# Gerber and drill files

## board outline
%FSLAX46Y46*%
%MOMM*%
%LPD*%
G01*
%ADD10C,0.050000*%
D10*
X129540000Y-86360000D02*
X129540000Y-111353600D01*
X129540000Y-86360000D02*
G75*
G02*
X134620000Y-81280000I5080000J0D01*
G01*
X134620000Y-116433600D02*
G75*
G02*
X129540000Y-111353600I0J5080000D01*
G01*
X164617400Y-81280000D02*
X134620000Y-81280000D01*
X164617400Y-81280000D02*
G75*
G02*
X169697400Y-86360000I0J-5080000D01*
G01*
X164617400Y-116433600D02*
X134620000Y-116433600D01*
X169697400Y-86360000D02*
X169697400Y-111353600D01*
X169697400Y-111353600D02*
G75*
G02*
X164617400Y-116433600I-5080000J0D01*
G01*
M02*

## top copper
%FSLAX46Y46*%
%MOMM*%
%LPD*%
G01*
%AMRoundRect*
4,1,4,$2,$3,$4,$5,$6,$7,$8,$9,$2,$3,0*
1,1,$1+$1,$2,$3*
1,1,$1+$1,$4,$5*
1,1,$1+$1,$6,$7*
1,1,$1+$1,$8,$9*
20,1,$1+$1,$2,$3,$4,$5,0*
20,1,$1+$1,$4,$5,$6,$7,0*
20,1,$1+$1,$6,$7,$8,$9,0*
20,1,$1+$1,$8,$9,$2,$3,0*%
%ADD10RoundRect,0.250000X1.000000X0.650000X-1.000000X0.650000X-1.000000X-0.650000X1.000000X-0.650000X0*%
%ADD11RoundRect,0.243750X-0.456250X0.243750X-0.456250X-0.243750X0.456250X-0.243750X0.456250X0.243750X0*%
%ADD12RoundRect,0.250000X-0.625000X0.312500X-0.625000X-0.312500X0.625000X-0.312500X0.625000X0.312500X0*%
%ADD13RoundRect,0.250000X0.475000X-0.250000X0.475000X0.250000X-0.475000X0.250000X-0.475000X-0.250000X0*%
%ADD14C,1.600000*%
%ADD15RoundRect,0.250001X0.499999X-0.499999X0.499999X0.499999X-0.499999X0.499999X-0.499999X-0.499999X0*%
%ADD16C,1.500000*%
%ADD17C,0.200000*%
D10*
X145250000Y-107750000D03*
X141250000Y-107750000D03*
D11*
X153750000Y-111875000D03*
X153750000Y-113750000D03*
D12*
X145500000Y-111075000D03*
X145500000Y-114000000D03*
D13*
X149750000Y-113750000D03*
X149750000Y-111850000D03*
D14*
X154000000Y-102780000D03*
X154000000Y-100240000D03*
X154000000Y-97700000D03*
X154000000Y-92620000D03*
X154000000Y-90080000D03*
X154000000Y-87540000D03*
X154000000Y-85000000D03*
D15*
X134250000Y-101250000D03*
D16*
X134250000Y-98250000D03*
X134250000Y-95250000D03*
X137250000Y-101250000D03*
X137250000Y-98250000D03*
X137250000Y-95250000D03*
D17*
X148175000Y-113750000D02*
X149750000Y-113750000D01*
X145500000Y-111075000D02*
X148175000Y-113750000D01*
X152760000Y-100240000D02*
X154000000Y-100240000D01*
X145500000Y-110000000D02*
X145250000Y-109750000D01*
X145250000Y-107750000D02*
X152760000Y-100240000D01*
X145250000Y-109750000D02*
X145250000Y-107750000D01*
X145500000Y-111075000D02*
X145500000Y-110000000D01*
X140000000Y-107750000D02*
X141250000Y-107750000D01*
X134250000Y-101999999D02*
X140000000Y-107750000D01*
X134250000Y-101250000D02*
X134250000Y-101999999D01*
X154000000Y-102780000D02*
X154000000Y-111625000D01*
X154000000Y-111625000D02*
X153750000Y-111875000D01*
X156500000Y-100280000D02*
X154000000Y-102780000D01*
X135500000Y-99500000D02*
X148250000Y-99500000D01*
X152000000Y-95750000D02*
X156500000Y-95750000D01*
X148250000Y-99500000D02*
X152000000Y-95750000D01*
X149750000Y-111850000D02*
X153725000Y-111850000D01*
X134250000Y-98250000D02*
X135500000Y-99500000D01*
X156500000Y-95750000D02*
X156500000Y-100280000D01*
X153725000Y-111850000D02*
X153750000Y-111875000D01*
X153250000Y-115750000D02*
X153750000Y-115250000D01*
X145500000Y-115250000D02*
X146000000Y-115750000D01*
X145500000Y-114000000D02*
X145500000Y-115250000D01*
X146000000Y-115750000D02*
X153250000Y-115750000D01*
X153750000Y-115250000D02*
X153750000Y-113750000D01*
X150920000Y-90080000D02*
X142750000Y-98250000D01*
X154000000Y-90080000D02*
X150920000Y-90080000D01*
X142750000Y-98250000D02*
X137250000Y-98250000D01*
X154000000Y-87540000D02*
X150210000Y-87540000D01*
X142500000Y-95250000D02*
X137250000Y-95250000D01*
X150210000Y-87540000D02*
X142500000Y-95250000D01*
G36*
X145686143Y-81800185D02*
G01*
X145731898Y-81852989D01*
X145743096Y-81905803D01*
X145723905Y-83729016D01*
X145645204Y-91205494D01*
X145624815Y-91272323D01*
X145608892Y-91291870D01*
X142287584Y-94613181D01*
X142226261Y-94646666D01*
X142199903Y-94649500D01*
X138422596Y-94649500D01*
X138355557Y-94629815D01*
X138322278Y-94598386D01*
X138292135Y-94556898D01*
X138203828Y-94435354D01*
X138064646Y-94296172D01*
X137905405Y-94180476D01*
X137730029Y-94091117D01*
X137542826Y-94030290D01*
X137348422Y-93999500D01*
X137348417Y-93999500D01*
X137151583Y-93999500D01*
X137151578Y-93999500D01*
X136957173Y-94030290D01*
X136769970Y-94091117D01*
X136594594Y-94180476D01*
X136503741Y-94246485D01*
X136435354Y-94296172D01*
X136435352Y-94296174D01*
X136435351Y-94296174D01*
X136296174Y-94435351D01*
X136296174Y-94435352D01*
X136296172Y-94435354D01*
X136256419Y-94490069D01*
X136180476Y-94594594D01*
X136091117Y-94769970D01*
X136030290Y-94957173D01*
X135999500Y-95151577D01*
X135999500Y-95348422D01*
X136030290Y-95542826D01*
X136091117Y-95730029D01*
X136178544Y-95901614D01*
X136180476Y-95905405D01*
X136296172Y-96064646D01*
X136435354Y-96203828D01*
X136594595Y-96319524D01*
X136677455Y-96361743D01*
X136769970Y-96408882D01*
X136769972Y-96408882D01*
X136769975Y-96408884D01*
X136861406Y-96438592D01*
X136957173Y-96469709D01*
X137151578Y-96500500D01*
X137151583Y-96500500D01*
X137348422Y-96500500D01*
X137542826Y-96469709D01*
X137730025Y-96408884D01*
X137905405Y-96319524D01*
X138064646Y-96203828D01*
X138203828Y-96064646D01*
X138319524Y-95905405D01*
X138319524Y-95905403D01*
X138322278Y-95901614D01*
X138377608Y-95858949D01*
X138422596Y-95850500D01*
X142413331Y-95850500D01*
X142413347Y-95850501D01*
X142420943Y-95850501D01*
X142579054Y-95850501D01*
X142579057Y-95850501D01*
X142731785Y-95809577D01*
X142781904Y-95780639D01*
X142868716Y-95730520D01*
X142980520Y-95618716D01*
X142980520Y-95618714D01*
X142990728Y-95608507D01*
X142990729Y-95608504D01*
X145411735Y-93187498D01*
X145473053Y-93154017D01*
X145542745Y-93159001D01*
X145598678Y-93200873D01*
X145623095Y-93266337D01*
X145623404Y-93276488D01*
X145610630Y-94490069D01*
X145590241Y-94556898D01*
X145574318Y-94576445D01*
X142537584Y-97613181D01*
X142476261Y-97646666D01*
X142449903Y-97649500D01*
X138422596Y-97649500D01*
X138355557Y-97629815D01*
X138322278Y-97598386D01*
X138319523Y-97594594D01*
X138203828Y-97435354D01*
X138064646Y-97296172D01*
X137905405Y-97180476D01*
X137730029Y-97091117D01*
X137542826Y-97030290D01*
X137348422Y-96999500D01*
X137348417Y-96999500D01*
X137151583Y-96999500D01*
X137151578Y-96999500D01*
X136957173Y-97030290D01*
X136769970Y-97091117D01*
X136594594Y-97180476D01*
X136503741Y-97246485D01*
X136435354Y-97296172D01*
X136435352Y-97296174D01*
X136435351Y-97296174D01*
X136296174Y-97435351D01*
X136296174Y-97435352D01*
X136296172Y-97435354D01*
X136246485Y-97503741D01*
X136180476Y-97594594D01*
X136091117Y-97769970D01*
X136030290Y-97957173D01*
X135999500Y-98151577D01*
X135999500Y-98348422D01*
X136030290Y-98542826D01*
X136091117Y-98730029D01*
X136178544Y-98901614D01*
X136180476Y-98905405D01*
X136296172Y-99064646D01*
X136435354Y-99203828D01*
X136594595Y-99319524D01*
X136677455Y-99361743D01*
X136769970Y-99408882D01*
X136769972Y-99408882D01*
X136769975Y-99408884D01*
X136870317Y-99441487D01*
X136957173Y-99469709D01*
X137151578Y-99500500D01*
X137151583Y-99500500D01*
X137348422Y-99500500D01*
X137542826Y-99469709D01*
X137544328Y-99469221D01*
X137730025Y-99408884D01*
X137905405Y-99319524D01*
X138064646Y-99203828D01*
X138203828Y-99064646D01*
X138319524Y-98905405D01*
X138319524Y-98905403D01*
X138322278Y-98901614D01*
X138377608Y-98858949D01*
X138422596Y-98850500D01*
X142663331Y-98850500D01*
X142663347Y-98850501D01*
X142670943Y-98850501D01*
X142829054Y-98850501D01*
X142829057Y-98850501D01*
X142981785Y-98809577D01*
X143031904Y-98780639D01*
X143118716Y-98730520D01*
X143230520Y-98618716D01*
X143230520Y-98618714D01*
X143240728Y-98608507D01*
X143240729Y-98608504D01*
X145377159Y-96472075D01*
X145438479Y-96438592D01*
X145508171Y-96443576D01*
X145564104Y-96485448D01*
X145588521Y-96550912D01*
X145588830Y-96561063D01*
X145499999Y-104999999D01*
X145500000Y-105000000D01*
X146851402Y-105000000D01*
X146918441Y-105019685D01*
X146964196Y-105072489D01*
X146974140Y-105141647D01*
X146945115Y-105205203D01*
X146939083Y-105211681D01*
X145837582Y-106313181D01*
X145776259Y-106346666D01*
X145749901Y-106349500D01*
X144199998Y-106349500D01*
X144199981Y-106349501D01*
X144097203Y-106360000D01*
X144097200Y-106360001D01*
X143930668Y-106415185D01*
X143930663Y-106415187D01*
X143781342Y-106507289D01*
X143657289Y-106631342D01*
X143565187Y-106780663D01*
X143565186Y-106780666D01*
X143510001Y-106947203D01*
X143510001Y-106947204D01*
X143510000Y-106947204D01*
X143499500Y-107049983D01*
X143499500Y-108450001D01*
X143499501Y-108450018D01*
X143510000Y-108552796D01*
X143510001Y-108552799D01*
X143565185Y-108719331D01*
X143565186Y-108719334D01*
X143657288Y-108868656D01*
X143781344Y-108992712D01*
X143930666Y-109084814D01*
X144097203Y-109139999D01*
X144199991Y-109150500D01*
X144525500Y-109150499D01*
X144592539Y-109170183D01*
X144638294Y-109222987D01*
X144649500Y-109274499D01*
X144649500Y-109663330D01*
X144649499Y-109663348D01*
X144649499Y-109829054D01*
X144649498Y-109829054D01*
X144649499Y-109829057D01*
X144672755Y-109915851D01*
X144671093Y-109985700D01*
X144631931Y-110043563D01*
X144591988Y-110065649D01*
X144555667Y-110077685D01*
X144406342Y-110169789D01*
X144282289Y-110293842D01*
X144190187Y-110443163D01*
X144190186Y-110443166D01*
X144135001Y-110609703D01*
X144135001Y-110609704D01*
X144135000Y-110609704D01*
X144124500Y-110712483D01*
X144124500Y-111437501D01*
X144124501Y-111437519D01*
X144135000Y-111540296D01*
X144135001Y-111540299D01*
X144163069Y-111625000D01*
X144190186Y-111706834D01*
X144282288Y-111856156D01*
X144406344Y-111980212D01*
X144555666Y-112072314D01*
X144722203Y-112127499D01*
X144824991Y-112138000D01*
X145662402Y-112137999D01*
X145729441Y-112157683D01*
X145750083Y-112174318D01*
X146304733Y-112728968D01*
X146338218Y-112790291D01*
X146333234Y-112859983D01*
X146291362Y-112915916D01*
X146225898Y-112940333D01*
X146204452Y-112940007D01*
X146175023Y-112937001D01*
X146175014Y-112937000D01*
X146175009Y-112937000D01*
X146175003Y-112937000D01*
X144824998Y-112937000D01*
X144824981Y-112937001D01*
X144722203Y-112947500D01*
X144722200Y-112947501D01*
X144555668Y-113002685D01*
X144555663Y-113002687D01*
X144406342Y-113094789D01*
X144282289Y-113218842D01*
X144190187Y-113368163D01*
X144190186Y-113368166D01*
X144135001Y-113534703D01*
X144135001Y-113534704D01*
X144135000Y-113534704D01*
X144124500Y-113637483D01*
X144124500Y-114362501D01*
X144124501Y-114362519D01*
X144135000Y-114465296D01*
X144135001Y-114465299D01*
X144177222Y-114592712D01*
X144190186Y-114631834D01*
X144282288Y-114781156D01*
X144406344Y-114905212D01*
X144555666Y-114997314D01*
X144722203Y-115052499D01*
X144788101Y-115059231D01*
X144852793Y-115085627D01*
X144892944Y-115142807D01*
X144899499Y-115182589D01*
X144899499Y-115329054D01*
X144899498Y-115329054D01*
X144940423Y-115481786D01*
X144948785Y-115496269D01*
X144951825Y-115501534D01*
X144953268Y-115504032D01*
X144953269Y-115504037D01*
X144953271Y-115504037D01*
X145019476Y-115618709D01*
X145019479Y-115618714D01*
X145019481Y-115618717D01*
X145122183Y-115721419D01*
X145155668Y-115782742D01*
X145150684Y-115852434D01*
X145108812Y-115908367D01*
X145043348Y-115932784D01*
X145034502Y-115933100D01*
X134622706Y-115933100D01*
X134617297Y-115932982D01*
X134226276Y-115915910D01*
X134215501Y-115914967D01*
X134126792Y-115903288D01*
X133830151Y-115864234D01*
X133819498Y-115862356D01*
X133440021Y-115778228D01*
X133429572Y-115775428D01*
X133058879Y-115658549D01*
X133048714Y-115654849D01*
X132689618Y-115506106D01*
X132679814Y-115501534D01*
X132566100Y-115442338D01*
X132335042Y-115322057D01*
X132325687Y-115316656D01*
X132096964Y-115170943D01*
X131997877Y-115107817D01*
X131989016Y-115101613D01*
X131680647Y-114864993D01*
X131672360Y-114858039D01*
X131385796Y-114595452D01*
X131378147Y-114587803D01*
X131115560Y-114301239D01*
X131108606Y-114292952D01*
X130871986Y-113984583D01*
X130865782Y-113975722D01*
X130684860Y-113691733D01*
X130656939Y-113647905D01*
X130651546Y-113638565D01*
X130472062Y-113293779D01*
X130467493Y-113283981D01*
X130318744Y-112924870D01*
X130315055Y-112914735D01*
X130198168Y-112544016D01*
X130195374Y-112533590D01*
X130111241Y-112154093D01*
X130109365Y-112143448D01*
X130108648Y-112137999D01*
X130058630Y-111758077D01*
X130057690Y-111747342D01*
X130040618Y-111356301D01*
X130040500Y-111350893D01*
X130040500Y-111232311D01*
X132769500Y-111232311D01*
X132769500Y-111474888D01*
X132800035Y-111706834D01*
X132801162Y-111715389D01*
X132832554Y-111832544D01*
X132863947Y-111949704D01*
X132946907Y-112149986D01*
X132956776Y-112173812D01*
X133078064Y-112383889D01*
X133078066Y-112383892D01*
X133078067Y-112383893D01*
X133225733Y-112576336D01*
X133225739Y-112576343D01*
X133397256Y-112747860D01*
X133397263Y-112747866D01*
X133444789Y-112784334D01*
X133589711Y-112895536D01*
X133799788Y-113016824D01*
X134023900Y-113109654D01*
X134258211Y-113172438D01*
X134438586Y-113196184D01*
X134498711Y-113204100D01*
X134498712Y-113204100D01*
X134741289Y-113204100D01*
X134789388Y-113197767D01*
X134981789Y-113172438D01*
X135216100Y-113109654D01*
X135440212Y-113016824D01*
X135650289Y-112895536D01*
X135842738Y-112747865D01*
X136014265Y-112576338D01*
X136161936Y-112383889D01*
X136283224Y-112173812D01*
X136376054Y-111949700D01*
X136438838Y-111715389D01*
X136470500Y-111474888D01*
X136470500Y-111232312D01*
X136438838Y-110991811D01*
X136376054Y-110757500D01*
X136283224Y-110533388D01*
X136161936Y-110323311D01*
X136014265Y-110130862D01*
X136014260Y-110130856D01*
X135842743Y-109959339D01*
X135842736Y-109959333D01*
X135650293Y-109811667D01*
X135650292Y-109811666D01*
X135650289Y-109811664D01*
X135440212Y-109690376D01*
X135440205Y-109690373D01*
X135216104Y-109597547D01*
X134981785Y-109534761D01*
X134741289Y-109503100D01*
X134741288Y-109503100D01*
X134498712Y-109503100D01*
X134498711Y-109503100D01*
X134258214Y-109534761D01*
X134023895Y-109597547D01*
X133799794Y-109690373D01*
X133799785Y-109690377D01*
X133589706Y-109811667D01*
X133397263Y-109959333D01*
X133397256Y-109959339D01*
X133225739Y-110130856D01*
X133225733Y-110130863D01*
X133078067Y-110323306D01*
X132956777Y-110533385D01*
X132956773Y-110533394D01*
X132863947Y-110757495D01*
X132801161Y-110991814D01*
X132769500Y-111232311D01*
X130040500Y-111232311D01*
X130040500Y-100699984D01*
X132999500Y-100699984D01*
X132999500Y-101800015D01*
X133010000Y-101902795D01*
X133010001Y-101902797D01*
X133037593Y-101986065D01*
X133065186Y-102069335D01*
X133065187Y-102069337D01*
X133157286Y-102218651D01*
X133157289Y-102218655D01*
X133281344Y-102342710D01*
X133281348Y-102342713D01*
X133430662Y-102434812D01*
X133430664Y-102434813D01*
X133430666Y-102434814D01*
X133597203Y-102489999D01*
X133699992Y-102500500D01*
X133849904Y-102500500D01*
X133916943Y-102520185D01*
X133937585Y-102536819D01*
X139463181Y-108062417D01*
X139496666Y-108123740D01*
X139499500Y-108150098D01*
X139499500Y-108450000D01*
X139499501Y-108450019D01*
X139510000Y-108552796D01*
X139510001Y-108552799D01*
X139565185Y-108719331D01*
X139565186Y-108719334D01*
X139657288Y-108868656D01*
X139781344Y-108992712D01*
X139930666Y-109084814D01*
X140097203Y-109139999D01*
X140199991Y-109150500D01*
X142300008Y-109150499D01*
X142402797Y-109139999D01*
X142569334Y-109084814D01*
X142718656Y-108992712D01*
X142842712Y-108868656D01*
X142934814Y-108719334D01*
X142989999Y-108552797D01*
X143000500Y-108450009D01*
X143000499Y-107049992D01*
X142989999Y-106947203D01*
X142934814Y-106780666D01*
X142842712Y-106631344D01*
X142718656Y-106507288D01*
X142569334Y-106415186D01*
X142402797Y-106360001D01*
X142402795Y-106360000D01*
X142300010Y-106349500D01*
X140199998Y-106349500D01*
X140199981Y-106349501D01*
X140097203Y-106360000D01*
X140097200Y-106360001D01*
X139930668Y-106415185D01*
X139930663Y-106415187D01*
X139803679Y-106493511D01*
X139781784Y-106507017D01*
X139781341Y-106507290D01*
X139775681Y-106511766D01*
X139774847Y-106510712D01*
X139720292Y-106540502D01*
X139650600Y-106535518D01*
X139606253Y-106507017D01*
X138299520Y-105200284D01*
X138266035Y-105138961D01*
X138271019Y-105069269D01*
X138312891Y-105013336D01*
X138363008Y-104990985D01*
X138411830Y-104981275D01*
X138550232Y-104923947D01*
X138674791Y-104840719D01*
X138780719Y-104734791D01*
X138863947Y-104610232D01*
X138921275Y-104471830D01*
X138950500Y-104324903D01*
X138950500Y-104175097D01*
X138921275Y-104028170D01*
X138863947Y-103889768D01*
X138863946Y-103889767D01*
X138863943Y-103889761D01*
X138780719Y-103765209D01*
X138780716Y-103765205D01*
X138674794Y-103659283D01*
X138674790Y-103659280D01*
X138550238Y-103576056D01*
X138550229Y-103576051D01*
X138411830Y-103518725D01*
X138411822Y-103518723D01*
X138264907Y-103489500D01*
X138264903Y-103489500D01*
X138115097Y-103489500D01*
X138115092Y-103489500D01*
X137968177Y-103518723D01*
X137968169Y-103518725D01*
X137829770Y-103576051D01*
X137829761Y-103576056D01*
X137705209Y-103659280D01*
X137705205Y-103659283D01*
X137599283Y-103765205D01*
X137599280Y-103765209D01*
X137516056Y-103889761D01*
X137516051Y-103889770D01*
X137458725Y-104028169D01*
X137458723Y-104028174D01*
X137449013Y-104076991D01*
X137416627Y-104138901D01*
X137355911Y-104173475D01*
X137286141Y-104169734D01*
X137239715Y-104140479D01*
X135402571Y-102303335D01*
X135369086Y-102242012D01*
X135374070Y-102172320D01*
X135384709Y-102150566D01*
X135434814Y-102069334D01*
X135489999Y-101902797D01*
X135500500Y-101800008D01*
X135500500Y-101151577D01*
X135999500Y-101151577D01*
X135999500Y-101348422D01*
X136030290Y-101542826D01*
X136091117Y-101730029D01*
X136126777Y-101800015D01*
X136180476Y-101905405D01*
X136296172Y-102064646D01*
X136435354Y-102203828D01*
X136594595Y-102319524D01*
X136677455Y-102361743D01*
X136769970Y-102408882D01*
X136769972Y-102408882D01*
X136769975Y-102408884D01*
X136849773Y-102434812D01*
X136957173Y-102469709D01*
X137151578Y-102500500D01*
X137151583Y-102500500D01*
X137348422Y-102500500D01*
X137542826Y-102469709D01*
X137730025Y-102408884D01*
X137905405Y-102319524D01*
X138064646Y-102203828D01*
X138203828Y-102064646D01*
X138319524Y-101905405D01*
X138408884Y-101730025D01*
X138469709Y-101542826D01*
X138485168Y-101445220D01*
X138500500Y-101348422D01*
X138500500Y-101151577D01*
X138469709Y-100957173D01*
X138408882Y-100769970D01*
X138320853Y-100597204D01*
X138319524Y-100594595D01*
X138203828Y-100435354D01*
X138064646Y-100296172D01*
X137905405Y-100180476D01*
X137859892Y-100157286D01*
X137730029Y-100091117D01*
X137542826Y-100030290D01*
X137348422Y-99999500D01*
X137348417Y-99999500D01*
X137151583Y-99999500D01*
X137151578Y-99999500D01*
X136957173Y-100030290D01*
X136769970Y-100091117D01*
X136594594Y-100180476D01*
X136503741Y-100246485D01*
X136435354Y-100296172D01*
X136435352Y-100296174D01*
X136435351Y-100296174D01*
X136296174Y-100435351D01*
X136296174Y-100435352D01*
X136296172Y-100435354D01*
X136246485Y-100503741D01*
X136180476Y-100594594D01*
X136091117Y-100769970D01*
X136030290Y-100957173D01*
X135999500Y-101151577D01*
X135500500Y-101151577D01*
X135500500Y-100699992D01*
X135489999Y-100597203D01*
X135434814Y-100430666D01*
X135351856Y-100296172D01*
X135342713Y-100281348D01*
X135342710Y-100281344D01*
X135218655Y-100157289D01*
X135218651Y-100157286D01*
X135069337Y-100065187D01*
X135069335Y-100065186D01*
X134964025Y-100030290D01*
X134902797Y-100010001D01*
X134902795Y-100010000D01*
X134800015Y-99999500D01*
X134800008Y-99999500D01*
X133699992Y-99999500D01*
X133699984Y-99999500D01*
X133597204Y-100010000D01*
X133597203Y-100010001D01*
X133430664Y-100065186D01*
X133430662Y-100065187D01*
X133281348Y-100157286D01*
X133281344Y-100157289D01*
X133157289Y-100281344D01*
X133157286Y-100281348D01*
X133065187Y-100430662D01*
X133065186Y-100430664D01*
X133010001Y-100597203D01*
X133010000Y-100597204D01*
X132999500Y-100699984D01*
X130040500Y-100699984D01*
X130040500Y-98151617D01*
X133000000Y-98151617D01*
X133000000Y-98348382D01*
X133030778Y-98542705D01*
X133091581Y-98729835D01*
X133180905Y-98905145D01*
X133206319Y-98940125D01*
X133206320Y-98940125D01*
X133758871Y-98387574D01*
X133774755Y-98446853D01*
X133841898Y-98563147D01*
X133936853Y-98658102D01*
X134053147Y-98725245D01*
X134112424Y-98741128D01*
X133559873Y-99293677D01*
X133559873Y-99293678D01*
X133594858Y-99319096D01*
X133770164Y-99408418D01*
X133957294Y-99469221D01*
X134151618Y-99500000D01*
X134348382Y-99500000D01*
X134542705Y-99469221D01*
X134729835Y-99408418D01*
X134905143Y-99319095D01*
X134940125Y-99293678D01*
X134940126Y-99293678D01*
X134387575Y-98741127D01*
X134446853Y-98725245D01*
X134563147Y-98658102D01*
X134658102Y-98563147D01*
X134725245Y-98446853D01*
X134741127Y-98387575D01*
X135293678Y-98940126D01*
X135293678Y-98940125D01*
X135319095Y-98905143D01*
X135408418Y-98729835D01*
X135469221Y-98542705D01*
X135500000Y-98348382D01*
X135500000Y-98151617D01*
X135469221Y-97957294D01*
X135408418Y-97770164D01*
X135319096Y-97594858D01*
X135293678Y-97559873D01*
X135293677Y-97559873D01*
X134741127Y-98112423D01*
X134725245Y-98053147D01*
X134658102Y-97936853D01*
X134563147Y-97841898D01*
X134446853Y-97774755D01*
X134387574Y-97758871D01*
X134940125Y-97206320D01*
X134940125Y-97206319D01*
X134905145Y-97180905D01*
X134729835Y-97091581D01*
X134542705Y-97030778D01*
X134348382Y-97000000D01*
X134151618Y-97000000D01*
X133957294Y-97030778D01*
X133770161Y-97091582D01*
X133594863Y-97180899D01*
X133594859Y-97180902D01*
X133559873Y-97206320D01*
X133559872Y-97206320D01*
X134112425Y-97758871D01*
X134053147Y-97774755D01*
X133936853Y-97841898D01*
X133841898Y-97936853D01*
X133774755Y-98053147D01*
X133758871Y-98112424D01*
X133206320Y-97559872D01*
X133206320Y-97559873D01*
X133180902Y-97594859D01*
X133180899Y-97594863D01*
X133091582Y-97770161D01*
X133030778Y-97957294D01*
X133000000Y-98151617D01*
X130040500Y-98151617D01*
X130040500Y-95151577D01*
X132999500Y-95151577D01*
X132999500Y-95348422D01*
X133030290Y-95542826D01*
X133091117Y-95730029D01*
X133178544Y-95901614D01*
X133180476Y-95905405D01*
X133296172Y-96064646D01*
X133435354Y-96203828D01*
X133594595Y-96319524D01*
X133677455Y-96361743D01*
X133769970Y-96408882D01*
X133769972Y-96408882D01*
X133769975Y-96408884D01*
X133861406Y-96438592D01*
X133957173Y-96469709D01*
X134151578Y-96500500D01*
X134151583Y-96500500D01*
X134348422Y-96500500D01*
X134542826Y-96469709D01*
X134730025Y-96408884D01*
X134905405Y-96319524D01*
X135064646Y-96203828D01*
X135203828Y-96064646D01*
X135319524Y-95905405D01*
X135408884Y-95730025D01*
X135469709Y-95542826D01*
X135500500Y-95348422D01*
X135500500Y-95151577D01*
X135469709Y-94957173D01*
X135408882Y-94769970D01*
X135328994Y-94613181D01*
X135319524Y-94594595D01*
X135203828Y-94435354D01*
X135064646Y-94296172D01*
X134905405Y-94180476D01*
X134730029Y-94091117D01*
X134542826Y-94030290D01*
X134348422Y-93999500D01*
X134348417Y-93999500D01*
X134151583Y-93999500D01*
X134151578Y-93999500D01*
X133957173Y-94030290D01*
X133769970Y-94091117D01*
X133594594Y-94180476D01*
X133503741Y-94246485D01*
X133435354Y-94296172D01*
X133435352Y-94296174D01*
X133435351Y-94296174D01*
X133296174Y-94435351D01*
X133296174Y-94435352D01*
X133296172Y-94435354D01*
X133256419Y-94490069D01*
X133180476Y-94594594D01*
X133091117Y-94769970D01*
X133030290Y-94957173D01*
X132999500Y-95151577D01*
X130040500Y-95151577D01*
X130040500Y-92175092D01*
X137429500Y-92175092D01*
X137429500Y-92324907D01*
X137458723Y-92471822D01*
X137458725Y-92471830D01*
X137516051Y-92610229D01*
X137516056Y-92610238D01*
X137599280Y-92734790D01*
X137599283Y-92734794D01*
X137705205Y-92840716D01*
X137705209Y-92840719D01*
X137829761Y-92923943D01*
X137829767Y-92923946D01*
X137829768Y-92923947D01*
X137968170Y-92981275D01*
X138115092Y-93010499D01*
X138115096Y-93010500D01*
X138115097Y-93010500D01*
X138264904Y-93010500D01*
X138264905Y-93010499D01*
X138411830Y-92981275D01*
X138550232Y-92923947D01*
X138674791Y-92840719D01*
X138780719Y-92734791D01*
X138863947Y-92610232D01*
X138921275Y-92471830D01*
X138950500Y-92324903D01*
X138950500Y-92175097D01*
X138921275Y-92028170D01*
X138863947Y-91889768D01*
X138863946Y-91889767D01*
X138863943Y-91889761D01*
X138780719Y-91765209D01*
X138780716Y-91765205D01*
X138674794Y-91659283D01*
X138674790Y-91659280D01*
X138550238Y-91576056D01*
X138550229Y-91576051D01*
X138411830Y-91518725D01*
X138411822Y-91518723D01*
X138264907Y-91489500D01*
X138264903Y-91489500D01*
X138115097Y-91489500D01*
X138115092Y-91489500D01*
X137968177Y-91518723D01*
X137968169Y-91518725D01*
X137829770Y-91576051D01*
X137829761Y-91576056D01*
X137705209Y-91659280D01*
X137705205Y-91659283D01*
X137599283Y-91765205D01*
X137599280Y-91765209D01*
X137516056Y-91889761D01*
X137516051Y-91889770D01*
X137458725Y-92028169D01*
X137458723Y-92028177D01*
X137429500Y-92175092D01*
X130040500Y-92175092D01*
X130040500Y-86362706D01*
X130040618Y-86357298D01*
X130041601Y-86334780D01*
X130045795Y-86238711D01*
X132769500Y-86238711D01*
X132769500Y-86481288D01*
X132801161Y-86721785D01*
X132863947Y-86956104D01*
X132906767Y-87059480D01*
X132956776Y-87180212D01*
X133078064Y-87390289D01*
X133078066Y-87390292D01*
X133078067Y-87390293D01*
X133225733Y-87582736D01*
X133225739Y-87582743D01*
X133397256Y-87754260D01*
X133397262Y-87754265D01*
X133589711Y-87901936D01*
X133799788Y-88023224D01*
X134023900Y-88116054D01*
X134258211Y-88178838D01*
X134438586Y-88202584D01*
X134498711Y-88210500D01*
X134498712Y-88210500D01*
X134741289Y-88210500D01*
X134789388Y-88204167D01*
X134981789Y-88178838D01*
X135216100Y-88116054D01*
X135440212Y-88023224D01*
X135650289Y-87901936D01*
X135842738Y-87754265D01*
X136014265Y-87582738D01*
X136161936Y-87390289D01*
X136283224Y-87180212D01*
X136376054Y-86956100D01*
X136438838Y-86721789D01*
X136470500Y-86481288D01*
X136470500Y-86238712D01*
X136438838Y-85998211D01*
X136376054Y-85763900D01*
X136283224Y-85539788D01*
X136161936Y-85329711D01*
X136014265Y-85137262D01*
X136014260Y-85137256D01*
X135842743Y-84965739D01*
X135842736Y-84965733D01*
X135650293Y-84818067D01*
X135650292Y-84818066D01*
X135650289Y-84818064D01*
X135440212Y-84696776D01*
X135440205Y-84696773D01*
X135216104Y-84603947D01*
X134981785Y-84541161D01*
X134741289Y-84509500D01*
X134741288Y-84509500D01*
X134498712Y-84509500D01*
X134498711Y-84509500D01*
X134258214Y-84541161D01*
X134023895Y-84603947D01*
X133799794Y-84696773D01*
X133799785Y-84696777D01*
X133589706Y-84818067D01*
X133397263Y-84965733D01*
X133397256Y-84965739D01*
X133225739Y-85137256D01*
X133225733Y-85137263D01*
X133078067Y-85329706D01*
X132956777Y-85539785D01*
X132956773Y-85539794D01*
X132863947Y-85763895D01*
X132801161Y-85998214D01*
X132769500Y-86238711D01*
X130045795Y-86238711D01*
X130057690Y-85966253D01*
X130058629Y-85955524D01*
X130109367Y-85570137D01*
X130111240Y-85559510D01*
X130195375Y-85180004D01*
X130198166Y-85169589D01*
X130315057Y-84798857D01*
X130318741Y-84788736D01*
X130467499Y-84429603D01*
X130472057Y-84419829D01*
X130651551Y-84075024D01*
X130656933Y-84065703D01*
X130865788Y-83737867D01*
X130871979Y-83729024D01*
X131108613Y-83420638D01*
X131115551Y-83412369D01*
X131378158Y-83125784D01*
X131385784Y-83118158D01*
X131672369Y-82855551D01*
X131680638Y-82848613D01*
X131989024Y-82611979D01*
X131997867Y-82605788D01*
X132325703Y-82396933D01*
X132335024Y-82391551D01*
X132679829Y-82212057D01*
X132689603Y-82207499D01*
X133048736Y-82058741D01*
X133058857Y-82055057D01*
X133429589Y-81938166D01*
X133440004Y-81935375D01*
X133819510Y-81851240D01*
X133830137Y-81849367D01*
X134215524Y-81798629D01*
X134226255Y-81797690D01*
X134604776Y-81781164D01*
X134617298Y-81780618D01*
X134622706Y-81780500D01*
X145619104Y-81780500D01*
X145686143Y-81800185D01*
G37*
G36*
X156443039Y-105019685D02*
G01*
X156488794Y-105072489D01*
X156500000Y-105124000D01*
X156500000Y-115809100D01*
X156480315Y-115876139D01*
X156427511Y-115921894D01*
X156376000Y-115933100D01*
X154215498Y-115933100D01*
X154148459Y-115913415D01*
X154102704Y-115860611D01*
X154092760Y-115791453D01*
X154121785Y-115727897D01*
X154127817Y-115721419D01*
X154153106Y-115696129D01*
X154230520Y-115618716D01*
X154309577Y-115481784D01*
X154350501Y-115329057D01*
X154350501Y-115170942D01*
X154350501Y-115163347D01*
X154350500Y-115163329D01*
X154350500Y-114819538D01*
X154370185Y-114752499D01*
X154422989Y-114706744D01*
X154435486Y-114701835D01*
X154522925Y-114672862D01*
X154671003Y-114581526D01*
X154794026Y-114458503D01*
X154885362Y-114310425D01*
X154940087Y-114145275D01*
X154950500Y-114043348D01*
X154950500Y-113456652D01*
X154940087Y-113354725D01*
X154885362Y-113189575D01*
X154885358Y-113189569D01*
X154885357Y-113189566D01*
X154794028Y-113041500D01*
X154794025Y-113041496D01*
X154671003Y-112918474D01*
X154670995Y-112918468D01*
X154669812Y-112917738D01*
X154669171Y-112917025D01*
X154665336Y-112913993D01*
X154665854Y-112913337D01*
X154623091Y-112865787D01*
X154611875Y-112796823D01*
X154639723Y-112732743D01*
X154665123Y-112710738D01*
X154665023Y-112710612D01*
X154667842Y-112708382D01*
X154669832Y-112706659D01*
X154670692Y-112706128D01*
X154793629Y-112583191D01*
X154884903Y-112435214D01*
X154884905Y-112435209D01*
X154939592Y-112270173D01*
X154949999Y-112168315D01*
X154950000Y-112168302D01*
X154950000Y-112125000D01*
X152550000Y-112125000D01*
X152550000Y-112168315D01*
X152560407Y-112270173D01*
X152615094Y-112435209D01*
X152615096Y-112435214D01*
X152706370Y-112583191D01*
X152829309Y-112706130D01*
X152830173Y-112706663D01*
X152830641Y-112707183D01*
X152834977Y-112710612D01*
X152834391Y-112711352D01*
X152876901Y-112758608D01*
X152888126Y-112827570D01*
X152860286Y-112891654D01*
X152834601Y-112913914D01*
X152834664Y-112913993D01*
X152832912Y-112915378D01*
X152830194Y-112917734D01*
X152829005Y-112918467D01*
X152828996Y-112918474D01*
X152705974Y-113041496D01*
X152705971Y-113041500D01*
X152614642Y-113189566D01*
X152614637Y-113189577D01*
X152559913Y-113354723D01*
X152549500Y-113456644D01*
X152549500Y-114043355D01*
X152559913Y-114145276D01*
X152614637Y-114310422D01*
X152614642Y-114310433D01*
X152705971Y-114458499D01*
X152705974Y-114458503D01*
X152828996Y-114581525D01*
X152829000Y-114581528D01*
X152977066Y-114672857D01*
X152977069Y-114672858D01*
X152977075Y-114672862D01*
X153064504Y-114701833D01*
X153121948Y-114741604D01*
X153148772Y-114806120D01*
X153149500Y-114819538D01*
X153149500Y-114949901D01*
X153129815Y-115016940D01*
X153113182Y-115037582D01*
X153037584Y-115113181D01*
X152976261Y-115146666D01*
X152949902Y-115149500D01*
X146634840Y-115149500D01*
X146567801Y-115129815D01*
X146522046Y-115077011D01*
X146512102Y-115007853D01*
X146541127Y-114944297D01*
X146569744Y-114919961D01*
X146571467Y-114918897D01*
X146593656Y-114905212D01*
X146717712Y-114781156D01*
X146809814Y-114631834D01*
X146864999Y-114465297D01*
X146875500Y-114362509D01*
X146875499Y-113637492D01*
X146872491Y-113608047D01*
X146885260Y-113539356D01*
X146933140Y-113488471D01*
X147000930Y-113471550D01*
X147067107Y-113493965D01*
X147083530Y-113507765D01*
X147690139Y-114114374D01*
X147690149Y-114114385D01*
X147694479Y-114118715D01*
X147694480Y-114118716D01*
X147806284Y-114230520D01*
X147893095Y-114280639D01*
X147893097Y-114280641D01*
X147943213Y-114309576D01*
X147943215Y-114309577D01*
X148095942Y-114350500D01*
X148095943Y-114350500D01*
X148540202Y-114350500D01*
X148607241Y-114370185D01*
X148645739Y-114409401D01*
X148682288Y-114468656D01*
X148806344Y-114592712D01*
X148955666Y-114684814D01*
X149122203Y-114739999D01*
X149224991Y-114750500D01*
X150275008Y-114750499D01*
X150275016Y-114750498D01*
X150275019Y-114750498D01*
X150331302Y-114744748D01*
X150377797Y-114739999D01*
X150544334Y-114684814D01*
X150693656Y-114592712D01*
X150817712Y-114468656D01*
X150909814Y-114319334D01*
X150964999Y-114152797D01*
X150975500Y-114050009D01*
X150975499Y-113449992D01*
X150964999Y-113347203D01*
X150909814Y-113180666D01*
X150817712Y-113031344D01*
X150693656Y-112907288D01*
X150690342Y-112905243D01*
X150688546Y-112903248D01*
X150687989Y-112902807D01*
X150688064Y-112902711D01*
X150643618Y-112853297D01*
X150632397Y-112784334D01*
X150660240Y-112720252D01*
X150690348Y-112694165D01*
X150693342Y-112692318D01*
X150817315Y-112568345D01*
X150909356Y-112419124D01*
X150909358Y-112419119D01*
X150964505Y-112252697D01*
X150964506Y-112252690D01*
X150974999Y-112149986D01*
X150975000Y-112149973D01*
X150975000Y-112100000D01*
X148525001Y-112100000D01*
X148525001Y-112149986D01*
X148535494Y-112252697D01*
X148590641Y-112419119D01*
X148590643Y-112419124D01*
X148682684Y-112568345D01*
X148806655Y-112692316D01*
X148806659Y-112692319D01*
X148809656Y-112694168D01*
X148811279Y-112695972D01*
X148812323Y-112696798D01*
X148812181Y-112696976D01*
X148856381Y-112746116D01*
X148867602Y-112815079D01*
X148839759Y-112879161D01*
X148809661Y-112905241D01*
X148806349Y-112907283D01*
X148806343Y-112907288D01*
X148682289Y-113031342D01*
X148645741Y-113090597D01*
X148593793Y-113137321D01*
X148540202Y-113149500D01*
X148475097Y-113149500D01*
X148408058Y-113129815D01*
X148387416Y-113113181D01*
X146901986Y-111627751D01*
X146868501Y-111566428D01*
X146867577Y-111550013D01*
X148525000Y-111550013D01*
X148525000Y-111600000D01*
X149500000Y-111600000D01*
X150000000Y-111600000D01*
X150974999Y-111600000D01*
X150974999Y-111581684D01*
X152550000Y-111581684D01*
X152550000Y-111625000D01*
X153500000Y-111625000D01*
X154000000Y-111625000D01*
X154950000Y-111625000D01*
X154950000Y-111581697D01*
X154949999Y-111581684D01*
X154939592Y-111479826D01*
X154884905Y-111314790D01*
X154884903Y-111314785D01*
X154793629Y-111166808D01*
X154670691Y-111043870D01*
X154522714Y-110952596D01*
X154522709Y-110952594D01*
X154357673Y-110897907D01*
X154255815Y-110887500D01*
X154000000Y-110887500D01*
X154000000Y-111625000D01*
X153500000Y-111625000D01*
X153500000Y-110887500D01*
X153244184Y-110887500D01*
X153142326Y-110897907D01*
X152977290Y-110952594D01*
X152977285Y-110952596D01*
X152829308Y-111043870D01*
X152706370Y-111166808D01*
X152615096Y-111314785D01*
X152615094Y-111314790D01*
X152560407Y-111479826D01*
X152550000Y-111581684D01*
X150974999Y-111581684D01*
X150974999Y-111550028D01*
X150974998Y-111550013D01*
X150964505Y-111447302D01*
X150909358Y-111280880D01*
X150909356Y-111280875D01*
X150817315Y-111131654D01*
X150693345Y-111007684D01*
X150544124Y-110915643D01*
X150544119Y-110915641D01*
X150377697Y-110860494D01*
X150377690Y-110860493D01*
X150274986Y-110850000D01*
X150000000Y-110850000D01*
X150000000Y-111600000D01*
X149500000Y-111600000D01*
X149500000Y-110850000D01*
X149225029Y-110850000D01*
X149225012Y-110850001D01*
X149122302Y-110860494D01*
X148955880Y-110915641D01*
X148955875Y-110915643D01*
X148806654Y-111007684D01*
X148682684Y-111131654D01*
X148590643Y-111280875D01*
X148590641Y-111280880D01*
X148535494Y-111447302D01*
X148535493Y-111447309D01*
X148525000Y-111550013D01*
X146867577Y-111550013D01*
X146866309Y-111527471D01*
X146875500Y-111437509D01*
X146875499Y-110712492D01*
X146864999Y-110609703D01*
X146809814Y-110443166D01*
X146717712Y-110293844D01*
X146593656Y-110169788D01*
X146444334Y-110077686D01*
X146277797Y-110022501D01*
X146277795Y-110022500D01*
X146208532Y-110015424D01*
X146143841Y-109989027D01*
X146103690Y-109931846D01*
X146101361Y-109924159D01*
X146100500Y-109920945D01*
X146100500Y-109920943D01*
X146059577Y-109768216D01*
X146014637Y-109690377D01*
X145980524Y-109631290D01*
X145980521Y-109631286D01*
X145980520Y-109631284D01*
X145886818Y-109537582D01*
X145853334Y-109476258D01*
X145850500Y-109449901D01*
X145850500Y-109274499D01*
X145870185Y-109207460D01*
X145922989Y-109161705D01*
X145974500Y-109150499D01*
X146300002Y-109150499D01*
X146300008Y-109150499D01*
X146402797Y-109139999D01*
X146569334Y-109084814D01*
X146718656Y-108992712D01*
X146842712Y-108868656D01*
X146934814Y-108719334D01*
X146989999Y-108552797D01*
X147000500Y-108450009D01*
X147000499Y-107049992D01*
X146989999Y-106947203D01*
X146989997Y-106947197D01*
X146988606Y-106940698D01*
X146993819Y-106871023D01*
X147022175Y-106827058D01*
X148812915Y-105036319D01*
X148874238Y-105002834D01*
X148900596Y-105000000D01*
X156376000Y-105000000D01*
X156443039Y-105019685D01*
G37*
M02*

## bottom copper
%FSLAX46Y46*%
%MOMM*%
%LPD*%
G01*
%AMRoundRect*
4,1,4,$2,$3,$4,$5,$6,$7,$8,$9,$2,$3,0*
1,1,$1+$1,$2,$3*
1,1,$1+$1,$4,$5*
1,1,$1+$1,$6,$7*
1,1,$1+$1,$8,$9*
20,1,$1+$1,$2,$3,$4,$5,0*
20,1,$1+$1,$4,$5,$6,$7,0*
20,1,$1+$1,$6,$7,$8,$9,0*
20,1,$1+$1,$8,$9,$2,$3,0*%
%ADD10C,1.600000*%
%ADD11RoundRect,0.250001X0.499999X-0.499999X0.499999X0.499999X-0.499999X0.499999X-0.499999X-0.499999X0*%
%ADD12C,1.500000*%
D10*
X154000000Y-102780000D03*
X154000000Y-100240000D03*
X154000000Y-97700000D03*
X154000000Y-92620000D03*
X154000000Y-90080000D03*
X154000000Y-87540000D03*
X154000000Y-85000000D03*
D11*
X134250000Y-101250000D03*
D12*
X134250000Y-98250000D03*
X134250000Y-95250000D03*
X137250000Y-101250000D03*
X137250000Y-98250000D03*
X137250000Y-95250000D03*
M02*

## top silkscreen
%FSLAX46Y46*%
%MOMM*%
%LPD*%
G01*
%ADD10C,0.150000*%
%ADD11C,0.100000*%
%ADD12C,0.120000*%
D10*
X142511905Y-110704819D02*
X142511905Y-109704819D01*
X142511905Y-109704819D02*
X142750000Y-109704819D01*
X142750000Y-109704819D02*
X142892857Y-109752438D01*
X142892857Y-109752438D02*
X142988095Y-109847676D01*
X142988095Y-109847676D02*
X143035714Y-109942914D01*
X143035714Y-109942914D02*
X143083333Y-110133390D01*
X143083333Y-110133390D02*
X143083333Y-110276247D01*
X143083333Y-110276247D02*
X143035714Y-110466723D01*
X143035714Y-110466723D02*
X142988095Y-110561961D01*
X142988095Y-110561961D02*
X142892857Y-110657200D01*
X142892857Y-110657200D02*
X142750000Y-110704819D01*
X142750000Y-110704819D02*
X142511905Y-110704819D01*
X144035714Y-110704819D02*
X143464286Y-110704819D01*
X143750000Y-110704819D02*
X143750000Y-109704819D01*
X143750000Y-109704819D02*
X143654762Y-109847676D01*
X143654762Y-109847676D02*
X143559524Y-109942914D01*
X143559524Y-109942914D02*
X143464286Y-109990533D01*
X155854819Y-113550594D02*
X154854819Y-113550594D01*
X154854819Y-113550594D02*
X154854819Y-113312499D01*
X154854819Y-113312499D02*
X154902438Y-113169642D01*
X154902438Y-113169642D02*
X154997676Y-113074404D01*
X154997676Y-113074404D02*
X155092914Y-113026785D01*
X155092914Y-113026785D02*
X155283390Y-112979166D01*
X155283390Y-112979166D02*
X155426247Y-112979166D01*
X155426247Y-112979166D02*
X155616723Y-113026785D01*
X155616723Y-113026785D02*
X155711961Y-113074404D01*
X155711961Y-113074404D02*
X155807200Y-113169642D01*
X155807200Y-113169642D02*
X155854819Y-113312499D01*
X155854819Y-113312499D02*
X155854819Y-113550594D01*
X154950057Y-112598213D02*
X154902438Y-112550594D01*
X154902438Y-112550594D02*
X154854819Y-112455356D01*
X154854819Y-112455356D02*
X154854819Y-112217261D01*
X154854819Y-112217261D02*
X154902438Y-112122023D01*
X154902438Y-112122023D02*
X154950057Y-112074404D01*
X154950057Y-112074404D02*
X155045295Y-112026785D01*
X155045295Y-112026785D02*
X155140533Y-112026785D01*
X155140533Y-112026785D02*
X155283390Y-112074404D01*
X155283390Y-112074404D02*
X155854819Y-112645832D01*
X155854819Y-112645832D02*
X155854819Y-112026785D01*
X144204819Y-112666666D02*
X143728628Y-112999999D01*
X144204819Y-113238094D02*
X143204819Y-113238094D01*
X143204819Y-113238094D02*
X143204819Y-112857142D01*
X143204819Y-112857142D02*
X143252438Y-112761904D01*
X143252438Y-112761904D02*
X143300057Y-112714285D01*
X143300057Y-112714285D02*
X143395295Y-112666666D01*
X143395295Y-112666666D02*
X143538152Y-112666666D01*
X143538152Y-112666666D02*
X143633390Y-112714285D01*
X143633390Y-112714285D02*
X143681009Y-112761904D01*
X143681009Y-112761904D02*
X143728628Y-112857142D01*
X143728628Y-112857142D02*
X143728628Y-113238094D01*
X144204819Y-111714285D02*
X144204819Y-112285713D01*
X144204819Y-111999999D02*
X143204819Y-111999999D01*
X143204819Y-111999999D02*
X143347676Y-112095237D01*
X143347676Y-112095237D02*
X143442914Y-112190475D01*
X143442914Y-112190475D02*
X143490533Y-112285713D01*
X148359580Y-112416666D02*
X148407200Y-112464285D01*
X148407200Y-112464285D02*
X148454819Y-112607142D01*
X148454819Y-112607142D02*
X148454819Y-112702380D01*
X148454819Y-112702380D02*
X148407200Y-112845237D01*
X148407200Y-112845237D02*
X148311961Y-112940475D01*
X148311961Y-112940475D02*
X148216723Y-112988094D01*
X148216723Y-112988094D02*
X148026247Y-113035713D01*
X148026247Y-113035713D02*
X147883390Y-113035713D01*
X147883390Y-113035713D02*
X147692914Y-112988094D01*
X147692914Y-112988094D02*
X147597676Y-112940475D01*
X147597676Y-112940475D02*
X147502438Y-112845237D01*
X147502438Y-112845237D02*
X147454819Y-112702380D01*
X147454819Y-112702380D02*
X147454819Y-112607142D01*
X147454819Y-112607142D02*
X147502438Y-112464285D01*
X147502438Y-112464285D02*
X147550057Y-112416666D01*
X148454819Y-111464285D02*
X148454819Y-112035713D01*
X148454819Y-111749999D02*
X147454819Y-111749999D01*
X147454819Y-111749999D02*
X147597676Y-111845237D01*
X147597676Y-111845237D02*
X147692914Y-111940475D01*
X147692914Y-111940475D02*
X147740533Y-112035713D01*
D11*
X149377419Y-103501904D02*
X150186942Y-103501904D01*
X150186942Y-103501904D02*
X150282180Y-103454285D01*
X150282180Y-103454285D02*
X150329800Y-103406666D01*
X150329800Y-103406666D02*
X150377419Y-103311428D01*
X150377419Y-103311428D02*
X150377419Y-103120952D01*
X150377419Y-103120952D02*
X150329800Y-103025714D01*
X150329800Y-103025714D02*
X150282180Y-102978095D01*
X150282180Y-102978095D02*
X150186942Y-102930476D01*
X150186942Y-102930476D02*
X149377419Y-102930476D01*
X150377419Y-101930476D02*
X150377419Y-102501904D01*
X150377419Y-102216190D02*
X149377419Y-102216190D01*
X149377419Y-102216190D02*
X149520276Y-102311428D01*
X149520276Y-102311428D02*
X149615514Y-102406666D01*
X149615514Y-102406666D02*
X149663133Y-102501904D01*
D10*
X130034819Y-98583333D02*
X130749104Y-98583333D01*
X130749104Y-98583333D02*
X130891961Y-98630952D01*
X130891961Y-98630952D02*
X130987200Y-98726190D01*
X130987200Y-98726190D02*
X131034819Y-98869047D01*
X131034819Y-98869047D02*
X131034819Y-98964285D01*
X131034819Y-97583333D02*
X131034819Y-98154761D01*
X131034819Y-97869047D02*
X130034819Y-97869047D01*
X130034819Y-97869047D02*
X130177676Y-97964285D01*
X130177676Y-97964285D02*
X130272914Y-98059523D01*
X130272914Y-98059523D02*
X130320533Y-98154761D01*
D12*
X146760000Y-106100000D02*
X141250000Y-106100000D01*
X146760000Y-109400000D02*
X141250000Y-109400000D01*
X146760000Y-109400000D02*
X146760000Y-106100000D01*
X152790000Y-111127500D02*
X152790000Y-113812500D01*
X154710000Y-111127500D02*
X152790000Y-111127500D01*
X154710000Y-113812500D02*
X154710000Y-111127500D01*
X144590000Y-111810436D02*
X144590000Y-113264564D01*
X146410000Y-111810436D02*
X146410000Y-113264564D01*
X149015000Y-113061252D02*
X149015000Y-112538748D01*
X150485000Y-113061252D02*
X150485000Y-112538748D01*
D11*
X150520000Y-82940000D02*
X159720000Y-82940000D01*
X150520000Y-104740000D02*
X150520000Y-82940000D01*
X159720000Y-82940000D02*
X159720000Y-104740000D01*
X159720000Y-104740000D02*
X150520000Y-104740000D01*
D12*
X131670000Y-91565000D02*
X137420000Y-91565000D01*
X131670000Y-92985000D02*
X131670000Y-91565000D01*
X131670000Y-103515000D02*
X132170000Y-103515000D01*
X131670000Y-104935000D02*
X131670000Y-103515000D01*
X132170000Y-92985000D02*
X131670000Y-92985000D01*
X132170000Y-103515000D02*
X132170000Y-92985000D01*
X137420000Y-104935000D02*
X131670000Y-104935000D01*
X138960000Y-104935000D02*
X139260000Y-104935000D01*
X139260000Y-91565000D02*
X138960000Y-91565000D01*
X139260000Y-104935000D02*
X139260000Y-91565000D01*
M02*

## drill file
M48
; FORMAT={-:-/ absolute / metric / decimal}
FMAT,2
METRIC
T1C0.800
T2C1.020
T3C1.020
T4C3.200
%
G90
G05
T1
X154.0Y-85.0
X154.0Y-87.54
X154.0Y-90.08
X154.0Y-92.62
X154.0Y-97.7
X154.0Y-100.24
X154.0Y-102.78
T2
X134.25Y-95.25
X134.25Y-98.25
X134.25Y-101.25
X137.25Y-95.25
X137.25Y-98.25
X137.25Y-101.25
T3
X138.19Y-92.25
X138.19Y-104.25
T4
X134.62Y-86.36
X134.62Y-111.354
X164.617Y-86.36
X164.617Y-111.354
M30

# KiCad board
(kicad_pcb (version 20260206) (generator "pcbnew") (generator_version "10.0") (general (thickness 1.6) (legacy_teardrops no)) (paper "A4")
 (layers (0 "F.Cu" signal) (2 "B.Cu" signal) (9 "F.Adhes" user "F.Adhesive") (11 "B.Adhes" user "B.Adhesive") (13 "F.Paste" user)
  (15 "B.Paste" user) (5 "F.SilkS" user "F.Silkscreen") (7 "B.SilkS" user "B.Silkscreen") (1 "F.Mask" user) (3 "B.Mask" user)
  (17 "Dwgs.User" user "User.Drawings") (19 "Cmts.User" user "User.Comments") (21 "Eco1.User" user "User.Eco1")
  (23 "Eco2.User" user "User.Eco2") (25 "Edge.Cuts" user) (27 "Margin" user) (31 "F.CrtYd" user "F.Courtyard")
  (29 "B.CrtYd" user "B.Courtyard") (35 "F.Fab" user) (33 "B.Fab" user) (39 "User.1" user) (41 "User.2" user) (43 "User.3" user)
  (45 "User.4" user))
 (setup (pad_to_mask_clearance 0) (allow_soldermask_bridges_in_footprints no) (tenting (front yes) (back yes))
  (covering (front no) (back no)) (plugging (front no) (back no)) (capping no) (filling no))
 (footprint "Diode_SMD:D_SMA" (layer "F.Cu") (at 143.25 107.75 180)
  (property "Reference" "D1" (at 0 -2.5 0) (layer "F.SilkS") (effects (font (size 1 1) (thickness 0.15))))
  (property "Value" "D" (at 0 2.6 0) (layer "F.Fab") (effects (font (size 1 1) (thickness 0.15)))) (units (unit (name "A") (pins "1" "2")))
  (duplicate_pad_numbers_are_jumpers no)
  (fp_line (start -3.51 1.65) (end 2 1.65) (stroke (width 0.12) (type solid)) (layer "F.SilkS"))
  (fp_line (start -3.51 -1.65) (end 2 -1.65) (stroke (width 0.12) (type solid)) (layer "F.SilkS"))
  (fp_line (start -3.51 -1.65) (end -3.51 1.65) (stroke (width 0.12) (type solid)) (layer "F.SilkS"))
  (pad "1" smd roundrect (at -2 0 180) (size 2.5 1.8) (layers "F.Cu" "F.Mask" "F.Paste") (roundrect_rratio 0.1388888889) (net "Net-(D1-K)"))
  (pad "2" smd roundrect (at 2 0 180) (size 2.5 1.8) (layers "F.Cu" "F.Mask" "F.Paste") (roundrect_rratio 0.1388888889) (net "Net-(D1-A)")))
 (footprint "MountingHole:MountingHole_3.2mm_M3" (layer "F.Cu") (at 134.62 86.36)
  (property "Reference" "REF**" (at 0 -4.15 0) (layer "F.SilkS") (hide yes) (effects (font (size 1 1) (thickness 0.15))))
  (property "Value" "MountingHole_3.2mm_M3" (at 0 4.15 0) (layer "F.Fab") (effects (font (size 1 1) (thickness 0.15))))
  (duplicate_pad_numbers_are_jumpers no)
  (pad "" np_thru_hole circle (at 0 0) (size 3.2 3.2) (drill 3.2) (layers "*.Cu" "*.Mask")))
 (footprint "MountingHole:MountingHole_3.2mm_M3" (layer "F.Cu") (at 134.62 111.3536)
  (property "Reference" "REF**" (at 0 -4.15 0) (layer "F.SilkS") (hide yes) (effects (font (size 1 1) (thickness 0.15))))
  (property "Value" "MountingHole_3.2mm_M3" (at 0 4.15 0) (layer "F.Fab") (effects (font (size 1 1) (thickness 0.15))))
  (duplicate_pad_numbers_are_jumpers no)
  (pad "" np_thru_hole circle (at 0 0) (size 3.2 3.2) (drill 3.2) (layers "*.Cu" "*.Mask")))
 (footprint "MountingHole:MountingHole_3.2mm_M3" (layer "F.Cu") (at 164.6174 86.36)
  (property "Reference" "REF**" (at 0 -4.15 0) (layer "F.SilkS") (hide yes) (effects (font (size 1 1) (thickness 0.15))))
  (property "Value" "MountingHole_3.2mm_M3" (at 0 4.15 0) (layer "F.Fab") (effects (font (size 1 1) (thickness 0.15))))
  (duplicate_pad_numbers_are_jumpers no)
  (pad "" np_thru_hole circle (at 0 0) (size 3.2 3.2) (drill 3.2) (layers "*.Cu" "*.Mask")))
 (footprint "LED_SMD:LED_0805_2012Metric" (layer "F.Cu") (at 153.75 112.8125 -90)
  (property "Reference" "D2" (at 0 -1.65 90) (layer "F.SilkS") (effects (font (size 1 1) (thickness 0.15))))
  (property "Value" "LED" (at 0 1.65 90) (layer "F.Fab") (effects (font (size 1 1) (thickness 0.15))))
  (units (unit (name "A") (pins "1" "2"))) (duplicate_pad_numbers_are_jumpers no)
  (fp_line (start -1.685 0.96) (end 1 0.96) (stroke (width 0.12) (type solid)) (layer "F.SilkS"))
  (fp_line (start -1.685 -0.96) (end -1.685 0.96) (stroke (width 0.12) (type solid)) (layer "F.SilkS"))
  (fp_line (start 1 -0.96) (end -1.685 -0.96) (stroke (width 0.12) (type solid)) (layer "F.SilkS"))
  (pad "1" smd roundrect (at -0.9375 0 270) (size 0.975 1.4) (layers "F.Cu" "F.Mask" "F.Paste") (roundrect_rratio 0.25) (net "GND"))
  (pad "2" smd roundrect (at 0.9375 0 270) (size 0.975 1.4) (layers "F.Cu" "F.Mask" "F.Paste") (roundrect_rratio 0.25) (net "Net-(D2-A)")))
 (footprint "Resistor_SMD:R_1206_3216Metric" (layer "F.Cu") (at 145.5 112.5375 -90)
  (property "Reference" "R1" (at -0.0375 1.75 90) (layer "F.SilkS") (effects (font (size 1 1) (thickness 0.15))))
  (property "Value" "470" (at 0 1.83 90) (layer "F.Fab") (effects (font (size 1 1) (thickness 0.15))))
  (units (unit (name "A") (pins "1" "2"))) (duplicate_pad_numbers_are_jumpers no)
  (fp_line (start -0.727064 0.91) (end 0.727064 0.91) (stroke (width 0.12) (type solid)) (layer "F.SilkS"))
  (fp_line (start -0.727064 -0.91) (end 0.727064 -0.91) (stroke (width 0.12) (type solid)) (layer "F.SilkS"))
  (pad "1" smd roundrect (at -1.4625 0 270) (size 1.125 1.75) (layers "F.Cu" "F.Mask" "F.Paste") (roundrect_rratio 0.222222)
   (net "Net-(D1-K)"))
  (pad "2" smd roundrect (at 1.4625 0 270) (size 1.125 1.75) (layers "F.Cu" "F.Mask" "F.Paste") (roundrect_rratio 0.222222)
   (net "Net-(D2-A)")))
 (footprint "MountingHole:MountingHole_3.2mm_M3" (layer "F.Cu") (at 164.6174 111.3536)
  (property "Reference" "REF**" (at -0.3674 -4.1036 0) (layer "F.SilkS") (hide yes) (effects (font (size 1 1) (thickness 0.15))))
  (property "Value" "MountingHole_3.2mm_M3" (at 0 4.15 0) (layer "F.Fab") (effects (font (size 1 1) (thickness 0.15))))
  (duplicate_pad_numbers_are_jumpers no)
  (pad "" np_thru_hole circle (at 0 0) (size 3.2 3.2) (drill 3.2) (layers "*.Cu" "*.Mask")))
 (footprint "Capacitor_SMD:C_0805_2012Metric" (layer "F.Cu") (at 149.75 112.8 90)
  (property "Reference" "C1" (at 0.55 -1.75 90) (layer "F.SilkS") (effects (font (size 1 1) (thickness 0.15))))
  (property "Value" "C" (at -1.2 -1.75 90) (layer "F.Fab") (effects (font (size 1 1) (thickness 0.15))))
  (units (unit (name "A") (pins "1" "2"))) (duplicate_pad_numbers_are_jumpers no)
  (fp_line (start -0.261252 -0.735) (end 0.261252 -0.735) (stroke (width 0.12) (type solid)) (layer "F.SilkS"))
  (fp_line (start -0.261252 0.735) (end 0.261252 0.735) (stroke (width 0.12) (type solid)) (layer "F.SilkS"))
  (pad "1" smd roundrect (at -0.95 0 90) (size 1 1.45) (layers "F.Cu" "F.Mask" "F.Paste") (roundrect_rratio 0.25) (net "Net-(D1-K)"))
  (pad "2" smd roundrect (at 0.95 0 90) (size 1 1.45) (layers "F.Cu" "F.Mask" "F.Paste") (roundrect_rratio 0.25) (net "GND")))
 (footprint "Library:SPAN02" (layer "F.Cu") (at 148.92 100.24 90)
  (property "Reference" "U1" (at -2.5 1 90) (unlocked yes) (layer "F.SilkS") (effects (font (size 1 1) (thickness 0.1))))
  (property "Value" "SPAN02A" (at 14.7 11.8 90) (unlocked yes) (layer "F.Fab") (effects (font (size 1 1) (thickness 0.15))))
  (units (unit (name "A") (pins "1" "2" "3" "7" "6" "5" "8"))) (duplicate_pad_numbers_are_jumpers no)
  (fp_line (start 17.3 1.6) (end 17.3 10.8) (stroke (width 0.1) (type default)) (layer "F.SilkS"))
  (fp_line (start -4.5 1.6) (end 17.3 1.6) (stroke (width 0.1) (type default)) (layer "F.SilkS"))
  (fp_line (start 17.3 10.8) (end -4.5 10.8) (stroke (width 0.1) (type default)) (layer "F.SilkS"))
  (fp_line (start -4.5 10.8) (end -4.5 1.6) (stroke (width 0.1) (type default)) (layer "F.SilkS"))
  (pad "1" thru_hole circle (at -2.54 5.08 90) (size 1.6 1.6) (drill 0.8) (layers "*.Cu" "*.Mask") (remove_unused_layers no) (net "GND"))
  (pad "2" thru_hole circle (at 0 5.08 90) (size 1.6 1.6) (drill 0.8) (layers "*.Cu" "*.Mask") (remove_unused_layers no) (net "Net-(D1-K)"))
  (pad "3" thru_hole circle (at 2.54 5.08 90) (size 1.6 1.6) (drill 0.8) (layers "*.Cu" "*.Mask") (remove_unused_layers no)
   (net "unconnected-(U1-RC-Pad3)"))
  (pad "5" thru_hole circle (at 7.62 5.08 90) (size 1.6 1.6) (drill 0.8) (layers "*.Cu" "*.Mask") (remove_unused_layers no)
   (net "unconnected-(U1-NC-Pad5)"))
  (pad "6" thru_hole circle (at 10.16 5.08 90) (size 1.6 1.6) (drill 0.8) (layers "*.Cu" "*.Mask") (remove_unused_layers no) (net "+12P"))
  (pad "7" thru_hole circle (at 12.7 5.08 90) (size 1.6 1.6) (drill 0.8) (layers "*.Cu" "*.Mask") (remove_unused_layers no) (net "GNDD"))
  (pad "8" thru_hole circle (at 15.24 5.08 90) (size 1.6 1.6) (drill 0.8) (layers "*.Cu" "*.Mask") (remove_unused_layers no)
   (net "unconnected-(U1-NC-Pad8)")))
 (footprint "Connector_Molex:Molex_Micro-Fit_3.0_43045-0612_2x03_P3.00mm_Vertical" (layer "F.Cu") (at 134.25 101.25 90)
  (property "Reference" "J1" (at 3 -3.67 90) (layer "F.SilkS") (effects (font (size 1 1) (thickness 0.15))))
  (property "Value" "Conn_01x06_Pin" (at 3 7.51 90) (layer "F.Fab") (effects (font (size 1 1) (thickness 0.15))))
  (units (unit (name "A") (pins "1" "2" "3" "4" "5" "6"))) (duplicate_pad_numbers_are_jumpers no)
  (fp_line (start 9.685 -2.58) (end 9.685 3.17) (stroke (width 0.12) (type solid)) (layer "F.SilkS"))
  (fp_line (start 8.265 -2.58) (end 9.685 -2.58) (stroke (width 0.12) (type solid)) (layer "F.SilkS"))
  (fp_line (start -2.265 -2.58) (end -2.265 -2.08) (stroke (width 0.12) (type solid)) (layer "F.SilkS"))
  (fp_line (start -3.685 -2.58) (end -2.265 -2.58) (stroke (width 0.12) (type solid)) (layer "F.SilkS"))
  (fp_line (start 8.265 -2.08) (end 8.265 -2.58) (stroke (width 0.12) (type solid)) (layer "F.SilkS"))
  (fp_line (start -2.265 -2.08) (end 8.265 -2.08) (stroke (width 0.12) (type solid)) (layer "F.SilkS"))
  (fp_line (start -3.685 3.17) (end -3.685 -2.58) (stroke (width 0.12) (type solid)) (layer "F.SilkS"))
  (fp_line (start -3.685 4.71) (end -3.685 5.01) (stroke (width 0.12) (type solid)) (layer "F.SilkS"))
  (fp_line (start 9.685 5.01) (end 9.685 4.71) (stroke (width 0.12) (type solid)) (layer "F.SilkS"))
  (fp_line (start -3.685 5.01) (end 9.685 5.01) (stroke (width 0.12) (type solid)) (layer "F.SilkS"))
  (pad "" np_thru_hole circle (at -3 3.94 90) (size 1.02 1.02) (drill 1.02) (layers "*.Cu" "*.Mask"))
  (pad "" np_thru_hole circle (at 9 3.94 90) (size 1.02 1.02) (drill 1.02) (layers "*.Cu" "*.Mask"))
  (pad "1" thru_hole roundrect (at 0 0 90) (size 1.5 1.5) (drill 1.02) (layers "*.Cu" "*.Mask") (remove_unused_layers no)
   (roundrect_rratio 0.166667) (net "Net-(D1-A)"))
  (pad "2" thru_hole circle (at 3 0 90) (size 1.5 1.5) (drill 1.02) (layers "*.Cu" "*.Mask") (remove_unused_layers no) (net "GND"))
  (pad "3" thru_hole circle (at 6 0 90) (size 1.5 1.5) (drill 1.02) (layers "*.Cu" "*.Mask") (remove_unused_layers no)
   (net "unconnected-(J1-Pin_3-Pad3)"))
  (pad "4" thru_hole circle (at 0 3 90) (size 1.5 1.5) (drill 1.02) (layers "*.Cu" "*.Mask") (remove_unused_layers no)
   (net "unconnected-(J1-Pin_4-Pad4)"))
  (pad "5" thru_hole circle (at 3 3 90) (size 1.5 1.5) (drill 1.02) (layers "*.Cu" "*.Mask") (remove_unused_layers no) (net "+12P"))
  (pad "6" thru_hole circle (at 6 3 90) (size 1.5 1.5) (drill 1.02) (layers "*.Cu" "*.Mask") (remove_unused_layers no) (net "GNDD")))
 (gr_line (start 129.54 86.36) (end 129.54 111.3536) (stroke (width 0.05) (type default)) (layer "Edge.Cuts"))
 (gr_arc (start 129.54 86.36) (mid 131.027898 82.767898) (end 134.62 81.28) (stroke (width 0.05) (type default)) (layer "Edge.Cuts"))
 (gr_arc (start 134.62 116.4336) (mid 131.027898 114.945702) (end 129.54 111.3536) (stroke (width 0.05) (type default)) (layer "Edge.Cuts"))
 (gr_line (start 164.6174 81.28) (end 134.62 81.28) (stroke (width 0.05) (type default)) (layer "Edge.Cuts"))
 (gr_arc (start 164.6174 81.28) (mid 168.209502 82.767898) (end 169.6974 86.36) (stroke (width 0.05) (type default)) (layer "Edge.Cuts"))
 (gr_line (start 164.6174 116.4336) (end 134.62 116.4336) (stroke (width 0.05) (type default)) (layer "Edge.Cuts"))
 (gr_line (start 169.6974 86.36) (end 169.6974 111.3536) (stroke (width 0.05) (type default)) (layer "Edge.Cuts"))
 (gr_arc (start 169.6974 111.3536) (mid 168.209502 114.945702) (end 164.6174 116.4336) (stroke (width 0.05) (type default))
  (layer "Edge.Cuts"))
 (segment (start 148.175 113.75) (end 149.75 113.75) (width 0.2) (layer "F.Cu") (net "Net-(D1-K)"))
 (segment (start 145.5 111.075) (end 148.175 113.75) (width 0.2) (layer "F.Cu") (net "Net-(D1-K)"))
 (segment (start 152.76 100.24) (end 154 100.24) (width 0.2) (layer "F.Cu") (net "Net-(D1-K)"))
 (segment (start 145.5 110) (end 145.25 109.75) (width 0.2) (layer "F.Cu") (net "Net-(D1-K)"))
 (segment (start 145.25 107.75) (end 152.76 100.24) (width 0.2) (layer "F.Cu") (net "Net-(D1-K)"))
 (segment (start 145.25 109.75) (end 145.25 107.75) (width 0.2) (layer "F.Cu") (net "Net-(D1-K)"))
 (segment (start 145.5 111.075) (end 145.5 110) (width 0.2) (layer "F.Cu") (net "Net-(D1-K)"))
 (segment (start 140 107.75) (end 141.25 107.75) (width 0.2) (layer "F.Cu") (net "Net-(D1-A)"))
 (segment (start 134.25 101.999999) (end 140 107.75) (width 0.2) (layer "F.Cu") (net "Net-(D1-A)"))
 (segment (start 134.25 101.25) (end 134.25 101.999999) (width 0.2) (layer "F.Cu") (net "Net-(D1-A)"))
 (segment (start 154 102.78) (end 154 111.625) (width 0.2) (layer "F.Cu") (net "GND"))
 (segment (start 154 111.625) (end 153.75 111.875) (width 0.2) (layer "F.Cu") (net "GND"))
 (segment (start 156.5 100.28) (end 154 102.78) (width 0.2) (layer "F.Cu") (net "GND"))
 (segment (start 135.5 99.5) (end 148.25 99.5) (width 0.2) (layer "F.Cu") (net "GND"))
 (segment (start 152 95.75) (end 156.5 95.75) (width 0.2) (layer "F.Cu") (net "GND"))
 (segment (start 148.25 99.5) (end 152 95.75) (width 0.2) (layer "F.Cu") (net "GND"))
 (segment (start 149.75 111.85) (end 153.725 111.85) (width 0.2) (layer "F.Cu") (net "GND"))
 (segment (start 134.25 98.25) (end 135.5 99.5) (width 0.2) (layer "F.Cu") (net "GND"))
 (segment (start 156.5 95.75) (end 156.5 100.28) (width 0.2) (layer "F.Cu") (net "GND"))
 (segment (start 153.725 111.85) (end 153.75 111.875) (width 0.2) (layer "F.Cu") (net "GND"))
 (segment (start 153.25 115.75) (end 153.75 115.25) (width 0.2) (layer "F.Cu") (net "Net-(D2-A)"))
 (segment (start 145.5 115.25) (end 146 115.75) (width 0.2) (layer "F.Cu") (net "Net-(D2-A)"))
 (segment (start 145.5 114) (end 145.5 115.25) (width 0.2) (layer "F.Cu") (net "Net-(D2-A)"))
 (segment (start 146 115.75) (end 153.25 115.75) (width 0.2) (layer "F.Cu") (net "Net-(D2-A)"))
 (segment (start 153.75 115.25) (end 153.75 113.75) (width 0.2) (layer "F.Cu") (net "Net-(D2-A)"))
 (segment (start 150.92 90.08) (end 142.75 98.25) (width 0.2) (layer "F.Cu") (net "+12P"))
 (segment (start 154 90.08) (end 150.92 90.08) (width 0.2) (layer "F.Cu") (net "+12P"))
 (segment (start 142.75 98.25) (end 137.25 98.25) (width 0.2) (layer "F.Cu") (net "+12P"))
 (segment (start 154 87.54) (end 150.21 87.54) (width 0.2) (layer "F.Cu") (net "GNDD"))
 (segment (start 142.5 95.25) (end 137.25 95.25) (width 0.2) (layer "F.Cu") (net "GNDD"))
 (segment (start 150.21 87.54) (end 142.5 95.25) (width 0.2) (layer "F.Cu") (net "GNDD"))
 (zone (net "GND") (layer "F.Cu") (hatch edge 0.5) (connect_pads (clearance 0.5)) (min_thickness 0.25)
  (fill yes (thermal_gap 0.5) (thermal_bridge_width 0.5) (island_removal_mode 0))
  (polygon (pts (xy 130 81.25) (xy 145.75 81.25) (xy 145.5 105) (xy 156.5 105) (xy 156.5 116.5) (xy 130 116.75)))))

